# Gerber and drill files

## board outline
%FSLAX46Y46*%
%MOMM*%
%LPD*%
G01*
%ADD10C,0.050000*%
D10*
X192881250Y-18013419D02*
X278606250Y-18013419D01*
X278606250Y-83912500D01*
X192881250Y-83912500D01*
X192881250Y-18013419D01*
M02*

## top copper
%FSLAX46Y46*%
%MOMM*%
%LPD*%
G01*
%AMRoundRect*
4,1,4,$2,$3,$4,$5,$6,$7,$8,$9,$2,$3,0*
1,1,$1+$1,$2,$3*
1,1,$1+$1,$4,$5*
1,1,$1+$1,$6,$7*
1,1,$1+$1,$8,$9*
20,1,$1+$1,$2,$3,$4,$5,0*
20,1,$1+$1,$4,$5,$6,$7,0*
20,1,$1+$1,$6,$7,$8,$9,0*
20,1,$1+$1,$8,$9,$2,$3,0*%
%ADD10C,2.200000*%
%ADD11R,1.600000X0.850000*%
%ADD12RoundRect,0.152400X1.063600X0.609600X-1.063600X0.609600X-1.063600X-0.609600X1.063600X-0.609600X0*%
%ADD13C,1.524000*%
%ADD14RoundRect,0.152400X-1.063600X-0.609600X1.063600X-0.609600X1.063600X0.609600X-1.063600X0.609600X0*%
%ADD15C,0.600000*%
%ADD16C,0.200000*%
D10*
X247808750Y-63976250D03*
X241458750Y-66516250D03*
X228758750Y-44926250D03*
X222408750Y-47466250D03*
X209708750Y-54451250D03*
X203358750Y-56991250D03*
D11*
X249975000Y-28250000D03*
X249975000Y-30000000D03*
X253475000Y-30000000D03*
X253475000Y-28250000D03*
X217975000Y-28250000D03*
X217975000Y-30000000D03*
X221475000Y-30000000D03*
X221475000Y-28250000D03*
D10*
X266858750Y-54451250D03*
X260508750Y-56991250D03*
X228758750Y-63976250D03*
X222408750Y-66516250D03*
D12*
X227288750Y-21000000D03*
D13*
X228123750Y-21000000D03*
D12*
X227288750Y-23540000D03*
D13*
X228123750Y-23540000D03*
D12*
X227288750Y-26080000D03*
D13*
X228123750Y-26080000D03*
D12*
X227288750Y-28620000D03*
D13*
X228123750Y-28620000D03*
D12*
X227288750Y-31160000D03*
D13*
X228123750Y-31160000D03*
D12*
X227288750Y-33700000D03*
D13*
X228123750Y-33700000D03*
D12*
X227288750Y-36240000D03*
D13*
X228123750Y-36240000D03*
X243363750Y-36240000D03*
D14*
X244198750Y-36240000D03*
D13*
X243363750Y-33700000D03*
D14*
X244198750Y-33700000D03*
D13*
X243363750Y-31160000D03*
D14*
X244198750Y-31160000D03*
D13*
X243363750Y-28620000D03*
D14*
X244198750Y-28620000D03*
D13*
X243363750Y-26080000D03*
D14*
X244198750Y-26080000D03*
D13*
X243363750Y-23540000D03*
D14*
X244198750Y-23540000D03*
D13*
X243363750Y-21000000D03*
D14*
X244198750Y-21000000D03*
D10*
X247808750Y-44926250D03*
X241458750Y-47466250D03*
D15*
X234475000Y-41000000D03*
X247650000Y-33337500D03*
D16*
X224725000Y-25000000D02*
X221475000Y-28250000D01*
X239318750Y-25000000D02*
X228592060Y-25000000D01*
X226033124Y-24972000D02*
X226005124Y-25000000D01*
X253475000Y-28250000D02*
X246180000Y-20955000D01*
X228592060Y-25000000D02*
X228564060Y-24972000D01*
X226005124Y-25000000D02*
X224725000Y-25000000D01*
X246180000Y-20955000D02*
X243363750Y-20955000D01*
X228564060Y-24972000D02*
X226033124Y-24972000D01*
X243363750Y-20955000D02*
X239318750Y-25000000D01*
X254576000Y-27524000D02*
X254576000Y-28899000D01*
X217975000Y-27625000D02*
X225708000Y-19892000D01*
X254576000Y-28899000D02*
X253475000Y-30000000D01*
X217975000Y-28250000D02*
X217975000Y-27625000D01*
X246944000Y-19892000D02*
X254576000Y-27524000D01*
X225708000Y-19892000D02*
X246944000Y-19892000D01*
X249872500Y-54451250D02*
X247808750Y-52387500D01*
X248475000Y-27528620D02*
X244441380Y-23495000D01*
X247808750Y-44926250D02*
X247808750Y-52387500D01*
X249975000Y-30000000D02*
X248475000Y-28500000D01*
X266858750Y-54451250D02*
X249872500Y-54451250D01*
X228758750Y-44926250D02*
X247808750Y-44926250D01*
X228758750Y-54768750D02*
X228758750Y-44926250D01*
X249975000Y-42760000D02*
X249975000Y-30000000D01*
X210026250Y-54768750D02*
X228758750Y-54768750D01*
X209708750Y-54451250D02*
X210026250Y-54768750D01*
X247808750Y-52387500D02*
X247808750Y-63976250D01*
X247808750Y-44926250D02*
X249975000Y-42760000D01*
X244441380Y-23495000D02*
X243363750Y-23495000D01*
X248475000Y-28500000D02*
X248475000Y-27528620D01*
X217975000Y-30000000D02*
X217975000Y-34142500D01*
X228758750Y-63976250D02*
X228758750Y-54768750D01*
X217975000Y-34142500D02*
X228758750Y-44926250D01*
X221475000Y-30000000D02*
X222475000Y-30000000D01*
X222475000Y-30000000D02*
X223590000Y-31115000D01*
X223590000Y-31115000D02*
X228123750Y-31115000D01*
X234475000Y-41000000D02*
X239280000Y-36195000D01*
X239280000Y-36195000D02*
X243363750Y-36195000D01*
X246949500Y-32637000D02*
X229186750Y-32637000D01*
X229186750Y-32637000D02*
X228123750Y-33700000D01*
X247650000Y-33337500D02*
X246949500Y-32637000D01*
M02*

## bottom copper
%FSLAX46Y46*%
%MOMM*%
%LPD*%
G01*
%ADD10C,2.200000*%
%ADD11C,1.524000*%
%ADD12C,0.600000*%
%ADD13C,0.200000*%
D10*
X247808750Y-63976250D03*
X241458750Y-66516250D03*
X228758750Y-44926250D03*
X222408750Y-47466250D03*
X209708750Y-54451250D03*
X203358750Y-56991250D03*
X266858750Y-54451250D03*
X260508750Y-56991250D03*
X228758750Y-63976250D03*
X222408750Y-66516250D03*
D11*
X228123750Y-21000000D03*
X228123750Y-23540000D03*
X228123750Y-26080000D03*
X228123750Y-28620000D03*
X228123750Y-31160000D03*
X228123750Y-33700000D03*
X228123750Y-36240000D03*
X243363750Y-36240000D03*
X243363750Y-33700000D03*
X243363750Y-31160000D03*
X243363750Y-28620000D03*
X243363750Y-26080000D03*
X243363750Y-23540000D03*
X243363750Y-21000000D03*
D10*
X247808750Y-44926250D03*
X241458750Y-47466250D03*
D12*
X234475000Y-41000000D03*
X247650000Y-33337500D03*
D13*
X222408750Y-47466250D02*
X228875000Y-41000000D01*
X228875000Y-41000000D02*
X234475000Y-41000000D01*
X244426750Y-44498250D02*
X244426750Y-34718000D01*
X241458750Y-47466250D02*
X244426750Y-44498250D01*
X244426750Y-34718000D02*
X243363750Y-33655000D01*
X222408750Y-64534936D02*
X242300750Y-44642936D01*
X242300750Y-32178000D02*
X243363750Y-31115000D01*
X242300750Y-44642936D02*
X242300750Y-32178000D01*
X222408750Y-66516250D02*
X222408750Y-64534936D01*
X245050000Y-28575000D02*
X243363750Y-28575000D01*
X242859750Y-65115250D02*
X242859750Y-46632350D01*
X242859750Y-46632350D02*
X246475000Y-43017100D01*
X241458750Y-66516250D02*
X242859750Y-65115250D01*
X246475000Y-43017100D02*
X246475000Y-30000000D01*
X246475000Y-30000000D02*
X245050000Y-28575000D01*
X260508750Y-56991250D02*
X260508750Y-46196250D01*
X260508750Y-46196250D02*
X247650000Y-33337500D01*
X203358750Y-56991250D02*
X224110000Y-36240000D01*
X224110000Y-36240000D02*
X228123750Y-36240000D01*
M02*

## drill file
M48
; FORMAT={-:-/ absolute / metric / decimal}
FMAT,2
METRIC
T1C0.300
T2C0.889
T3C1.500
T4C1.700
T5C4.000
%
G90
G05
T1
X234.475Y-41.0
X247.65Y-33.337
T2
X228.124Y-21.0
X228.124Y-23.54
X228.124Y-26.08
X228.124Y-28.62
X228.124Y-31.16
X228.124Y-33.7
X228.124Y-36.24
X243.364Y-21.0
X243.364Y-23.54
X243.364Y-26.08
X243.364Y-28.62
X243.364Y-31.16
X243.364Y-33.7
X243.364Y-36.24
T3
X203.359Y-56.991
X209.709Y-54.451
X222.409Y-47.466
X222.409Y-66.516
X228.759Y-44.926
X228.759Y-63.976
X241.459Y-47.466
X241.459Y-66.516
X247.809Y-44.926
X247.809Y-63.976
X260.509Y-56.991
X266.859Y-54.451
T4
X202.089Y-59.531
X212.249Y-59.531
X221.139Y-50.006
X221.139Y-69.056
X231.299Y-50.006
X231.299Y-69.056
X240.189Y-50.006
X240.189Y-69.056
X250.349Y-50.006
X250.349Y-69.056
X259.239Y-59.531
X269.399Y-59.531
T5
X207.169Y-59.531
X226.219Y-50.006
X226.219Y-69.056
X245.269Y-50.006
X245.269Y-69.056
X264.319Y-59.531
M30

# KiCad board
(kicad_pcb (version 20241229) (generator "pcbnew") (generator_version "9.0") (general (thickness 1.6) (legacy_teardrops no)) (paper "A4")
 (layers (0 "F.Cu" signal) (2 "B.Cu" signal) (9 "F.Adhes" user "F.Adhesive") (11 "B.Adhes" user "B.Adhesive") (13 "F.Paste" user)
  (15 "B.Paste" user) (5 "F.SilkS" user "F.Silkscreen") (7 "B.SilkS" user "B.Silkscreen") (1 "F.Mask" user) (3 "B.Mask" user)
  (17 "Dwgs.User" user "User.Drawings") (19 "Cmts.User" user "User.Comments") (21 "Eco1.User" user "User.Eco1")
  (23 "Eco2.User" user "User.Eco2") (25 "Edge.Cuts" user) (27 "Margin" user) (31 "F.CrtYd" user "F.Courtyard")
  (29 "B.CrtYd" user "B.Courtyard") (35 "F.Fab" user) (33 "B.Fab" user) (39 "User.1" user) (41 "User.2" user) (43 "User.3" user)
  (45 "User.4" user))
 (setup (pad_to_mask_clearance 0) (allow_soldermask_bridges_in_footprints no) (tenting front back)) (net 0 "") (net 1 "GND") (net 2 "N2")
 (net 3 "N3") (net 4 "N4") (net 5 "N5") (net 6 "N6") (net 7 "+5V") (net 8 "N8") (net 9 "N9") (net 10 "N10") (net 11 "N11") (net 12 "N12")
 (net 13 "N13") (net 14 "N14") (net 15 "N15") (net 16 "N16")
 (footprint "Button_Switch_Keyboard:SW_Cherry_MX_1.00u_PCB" (layer "F.Cu") (at 247.80875 63.97625)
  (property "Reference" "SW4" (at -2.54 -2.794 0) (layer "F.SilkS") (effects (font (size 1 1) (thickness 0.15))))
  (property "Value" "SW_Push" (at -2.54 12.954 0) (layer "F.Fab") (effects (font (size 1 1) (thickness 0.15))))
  (pad "" np_thru_hole circle (at -7.62 5.08) (size 1.7 1.7) (drill 1.7) (layers "*.Cu" "*.Mask"))
  (pad "" np_thru_hole circle (at -2.54 5.08) (size 4 4) (drill 4) (layers "*.Cu" "*.Mask"))
  (pad "" np_thru_hole circle (at 2.54 5.08) (size 1.7 1.7) (drill 1.7) (layers "*.Cu" "*.Mask"))
  (pad "1" thru_hole circle (at 0 0) (size 2.2 2.2) (drill 1.5) (layers "*.Cu" "*.Mask") (remove_unused_layers no) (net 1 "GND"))
  (pad "2" thru_hole circle (at -6.35 2.54) (size 2.2 2.2) (drill 1.5) (layers "*.Cu" "*.Mask") (remove_unused_layers no) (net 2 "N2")))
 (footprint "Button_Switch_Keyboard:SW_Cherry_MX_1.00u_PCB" (layer "F.Cu") (at 228.75875 44.92625)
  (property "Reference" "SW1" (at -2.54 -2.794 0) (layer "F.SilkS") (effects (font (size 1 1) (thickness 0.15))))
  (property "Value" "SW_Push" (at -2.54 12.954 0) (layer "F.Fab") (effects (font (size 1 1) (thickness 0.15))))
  (pad "" np_thru_hole circle (at -7.62 5.08) (size 1.7 1.7) (drill 1.7) (layers "*.Cu" "*.Mask"))
  (pad "" np_thru_hole circle (at -2.54 5.08) (size 4 4) (drill 4) (layers "*.Cu" "*.Mask"))
  (pad "" np_thru_hole circle (at 2.54 5.08) (size 1.7 1.7) (drill 1.7) (layers "*.Cu" "*.Mask"))
  (pad "1" thru_hole circle (at 0 0) (size 2.2 2.2) (drill 1.5) (layers "*.Cu" "*.Mask") (remove_unused_layers no) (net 1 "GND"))
  (pad "2" thru_hole circle (at -6.35 2.54) (size 2.2 2.2) (drill 1.5) (layers "*.Cu" "*.Mask") (remove_unused_layers no) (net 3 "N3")))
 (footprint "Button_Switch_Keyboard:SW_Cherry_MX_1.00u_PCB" (layer "F.Cu") (at 209.70875 54.45125)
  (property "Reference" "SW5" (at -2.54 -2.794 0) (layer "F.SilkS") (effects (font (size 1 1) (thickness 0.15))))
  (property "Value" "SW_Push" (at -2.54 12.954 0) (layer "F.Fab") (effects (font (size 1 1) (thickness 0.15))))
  (pad "" np_thru_hole circle (at -7.62 5.08) (size 1.7 1.7) (drill 1.7) (layers "*.Cu" "*.Mask"))
  (pad "" np_thru_hole circle (at -2.54 5.08) (size 4 4) (drill 4) (layers "*.Cu" "*.Mask"))
  (pad "" np_thru_hole circle (at 2.54 5.08) (size 1.7 1.7) (drill 1.7) (layers "*.Cu" "*.Mask"))
  (pad "1" thru_hole circle (at 0 0) (size 2.2 2.2) (drill 1.5) (layers "*.Cu" "*.Mask") (remove_unused_layers no) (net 1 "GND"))
  (pad "2" thru_hole circle (at -6.35 2.54) (size 2.2 2.2) (drill 1.5) (layers "*.Cu" "*.Mask") (remove_unused_layers no) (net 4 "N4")))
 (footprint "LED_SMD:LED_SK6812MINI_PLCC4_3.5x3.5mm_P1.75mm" (layer "F.Cu") (at 251.725 29.125)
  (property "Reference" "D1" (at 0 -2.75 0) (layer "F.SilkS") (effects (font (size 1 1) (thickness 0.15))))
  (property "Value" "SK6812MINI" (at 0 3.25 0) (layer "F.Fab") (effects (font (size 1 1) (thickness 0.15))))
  (pad "1" smd rect (at -1.75 -0.875) (size 1.6 0.85) (layers "F.Cu" "F.Mask" "F.Paste") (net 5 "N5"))
  (pad "2" smd rect (at -1.75 0.875) (size 1.6 0.85) (layers "F.Cu" "F.Mask" "F.Paste") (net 1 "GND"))
  (pad "3" smd rect (at 1.75 0.875) (size 1.6 0.85) (layers "F.Cu" "F.Mask" "F.Paste") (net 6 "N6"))
  (pad "4" smd rect (at 1.75 -0.875) (size 1.6 0.85) (layers "F.Cu" "F.Mask" "F.Paste") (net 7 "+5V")))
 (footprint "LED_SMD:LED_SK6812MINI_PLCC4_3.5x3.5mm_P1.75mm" (layer "F.Cu") (at 219.725 29.125)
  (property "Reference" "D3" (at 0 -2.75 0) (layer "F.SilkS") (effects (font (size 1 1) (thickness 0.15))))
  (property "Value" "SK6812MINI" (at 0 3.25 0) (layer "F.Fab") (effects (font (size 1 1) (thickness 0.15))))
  (pad "1" smd rect (at -1.75 -0.875) (size 1.6 0.85) (layers "F.Cu" "F.Mask" "F.Paste") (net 6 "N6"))
  (pad "2" smd rect (at -1.75 0.875) (size 1.6 0.85) (layers "F.Cu" "F.Mask" "F.Paste") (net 1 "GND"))
  (pad "3" smd rect (at 1.75 0.875) (size 1.6 0.85) (layers "F.Cu" "F.Mask" "F.Paste") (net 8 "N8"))
  (pad "4" smd rect (at 1.75 -0.875) (size 1.6 0.85) (layers "F.Cu" "F.Mask" "F.Paste") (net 7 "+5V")))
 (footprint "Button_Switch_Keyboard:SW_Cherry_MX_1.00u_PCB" (layer "F.Cu") (at 266.85875 54.45125)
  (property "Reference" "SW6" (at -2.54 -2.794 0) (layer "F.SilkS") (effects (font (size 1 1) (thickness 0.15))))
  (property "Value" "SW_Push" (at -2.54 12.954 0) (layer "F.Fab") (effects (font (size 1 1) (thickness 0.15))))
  (pad "" np_thru_hole circle (at -7.62 5.08) (size 1.7 1.7) (drill 1.7) (layers "*.Cu" "*.Mask"))
  (pad "" np_thru_hole circle (at -2.54 5.08) (size 4 4) (drill 4) (layers "*.Cu" "*.Mask"))
  (pad "" np_thru_hole circle (at 2.54 5.08) (size 1.7 1.7) (drill 1.7) (layers "*.Cu" "*.Mask"))
  (pad "1" thru_hole circle (at 0 0) (size 2.2 2.2) (drill 1.5) (layers "*.Cu" "*.Mask") (remove_unused_layers no) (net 1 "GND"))
  (pad "2" thru_hole circle (at -6.35 2.54) (size 2.2 2.2) (drill 1.5) (layers "*.Cu" "*.Mask") (remove_unused_layers no) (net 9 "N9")))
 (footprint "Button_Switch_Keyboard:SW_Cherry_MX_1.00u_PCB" (layer "F.Cu") (at 228.75875 63.97625)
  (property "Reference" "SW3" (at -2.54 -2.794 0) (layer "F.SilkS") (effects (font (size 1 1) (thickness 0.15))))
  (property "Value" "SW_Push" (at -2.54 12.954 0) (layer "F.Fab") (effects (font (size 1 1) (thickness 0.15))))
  (pad "" np_thru_hole circle (at -7.62 5.08) (size 1.7 1.7) (drill 1.7) (layers "*.Cu" "*.Mask"))
  (pad "" np_thru_hole circle (at -2.54 5.08) (size 4 4) (drill 4) (layers "*.Cu" "*.Mask"))
  (pad "" np_thru_hole circle (at 2.54 5.08) (size 1.7 1.7) (drill 1.7) (layers "*.Cu" "*.Mask"))
  (pad "1" thru_hole circle (at 0 0) (size 2.2 2.2) (drill 1.5) (layers "*.Cu" "*.Mask") (remove_unused_layers no) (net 1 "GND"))
  (pad "2" thru_hole circle (at -6.35 2.54) (size 2.2 2.2) (drill 1.5) (layers "*.Cu" "*.Mask") (remove_unused_layers no) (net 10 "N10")))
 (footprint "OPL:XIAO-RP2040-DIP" (layer "F.Cu") (at 235.74375 28.62)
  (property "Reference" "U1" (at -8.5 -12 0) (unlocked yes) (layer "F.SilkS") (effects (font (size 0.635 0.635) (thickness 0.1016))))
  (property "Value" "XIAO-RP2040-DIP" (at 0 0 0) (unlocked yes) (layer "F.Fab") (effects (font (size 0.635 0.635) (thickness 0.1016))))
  (pad "1" smd roundrect (at -8.455 -7.62 180) (size 2.432 1.524) (layers "F.Cu" "F.Mask") (roundrect_rratio 0.1) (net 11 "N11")
   (thermal_bridge_angle 45))
  (pad "1" thru_hole circle (at -7.62 -7.62 180) (size 1.524 1.524) (drill 0.889) (layers "*.Cu" "*.Mask") (remove_unused_layers no)
   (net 11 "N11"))
  (pad "2" smd roundrect (at -8.455 -5.08 180) (size 2.432 1.524) (layers "F.Cu" "F.Mask") (roundrect_rratio 0.1) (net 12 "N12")
   (thermal_bridge_angle 45))
  (pad "2" thru_hole circle (at -7.62 -5.08 180) (size 1.524 1.524) (drill 0.889) (layers "*.Cu" "*.Mask") (remove_unused_layers no)
   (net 12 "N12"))
  (pad "3" smd roundrect (at -8.455 -2.54 180) (size 2.432 1.524) (layers "F.Cu" "F.Mask") (roundrect_rratio 0.1) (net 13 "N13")
   (thermal_bridge_angle 45))
  (pad "3" thru_hole circle (at -7.62 -2.54 180) (size 1.524 1.524) (drill 0.889) (layers "*.Cu" "*.Mask") (remove_unused_layers no)
   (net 13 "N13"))
  (pad "4" smd roundrect (at -8.455 0 180) (size 2.432 1.524) (layers "F.Cu" "F.Mask") (roundrect_rratio 0.1) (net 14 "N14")
   (thermal_bridge_angle 45))
  (pad "4" thru_hole circle (at -7.62 0 180) (size 1.524 1.524) (drill 0.889) (layers "*.Cu" "*.Mask") (remove_unused_layers no)
   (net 14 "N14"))
  (pad "5" smd roundrect (at -8.455 2.54 180) (size 2.432 1.524) (layers "F.Cu" "F.Mask") (roundrect_rratio 0.1) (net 8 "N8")
   (thermal_bridge_angle 45))
  (pad "5" thru_hole circle (at -7.62 2.54 180) (size 1.524 1.524) (drill 0.889) (layers "*.Cu" "*.Mask") (remove_unused_layers no)
   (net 8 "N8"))
  (pad "6" smd roundrect (at -8.455 5.08 180) (size 2.432 1.524) (layers "F.Cu" "F.Mask") (roundrect_rratio 0.1) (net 9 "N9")
   (thermal_bridge_angle 45))
  (pad "6" thru_hole circle (at -7.62 5.08 180) (size 1.524 1.524) (drill 0.889) (layers "*.Cu" "*.Mask") (remove_unused_layers no)
   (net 9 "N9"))
  (pad "7" smd roundrect (at -8.455 7.62 180) (size 2.432 1.524) (layers "F.Cu" "F.Mask") (roundrect_rratio 0.1) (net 4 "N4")
   (thermal_bridge_angle 45))
  (pad "7" thru_hole circle (at -7.62 7.62 180) (size 1.524 1.524) (drill 0.889) (layers "*.Cu" "*.Mask") (remove_unused_layers no)
   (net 4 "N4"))
  (pad "8" thru_hole circle (at 7.62 7.62) (size 1.524 1.524) (drill 0.889) (layers "*.Cu" "*.Mask") (remove_unused_layers no) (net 3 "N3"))
  (pad "8" smd roundrect (at 8.455 7.62) (size 2.432 1.524) (layers "F.Cu" "F.Mask") (roundrect_rratio 0.1) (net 3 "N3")
   (thermal_bridge_angle 45))
  (pad "9" thru_hole circle (at 7.62 5.08) (size 1.524 1.524) (drill 0.889) (layers "*.Cu" "*.Mask") (remove_unused_layers no)
   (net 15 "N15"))
  (pad "9" smd roundrect (at 8.455 5.08) (size 2.432 1.524) (layers "F.Cu" "F.Mask") (roundrect_rratio 0.1) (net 15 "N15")
   (thermal_bridge_angle 45))
  (pad "10" thru_hole circle (at 7.62 2.54) (size 1.524 1.524) (drill 0.889) (layers "*.Cu" "*.Mask") (remove_unused_layers no)
   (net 10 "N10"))
  (pad "10" smd roundrect (at 8.455 2.54) (size 2.432 1.524) (layers "F.Cu" "F.Mask") (roundrect_rratio 0.1) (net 10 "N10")
   (thermal_bridge_angle 45))
  (pad "11" thru_hole circle (at 7.62 0) (size 1.524 1.524) (drill 0.889) (layers "*.Cu" "*.Mask") (remove_unused_layers no) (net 2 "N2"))
  (pad "11" smd roundrect (at 8.455 0) (size 2.432 1.524) (layers "F.Cu" "F.Mask") (roundrect_rratio 0.1) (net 2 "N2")
   (thermal_bridge_angle 45))
  (pad "12" thru_hole circle (at 7.62 -2.54) (size 1.524 1.524) (drill 0.889) (layers "*.Cu" "*.Mask") (remove_unused_layers no)
   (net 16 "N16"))
  (pad "12" smd roundrect (at 8.455 -2.54) (size 2.432 1.524) (layers "F.Cu" "F.Mask") (roundrect_rratio 0.1) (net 16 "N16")
   (thermal_bridge_angle 45))
  (pad "13" thru_hole circle (at 7.62 -5.08) (size 1.524 1.524) (drill 0.889) (layers "*.Cu" "*.Mask") (remove_unused_layers no)
   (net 1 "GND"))
  (pad "13" smd roundrect (at 8.455 -5.08) (size 2.432 1.524) (layers "F.Cu" "F.Mask") (roundrect_rratio 0.1) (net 1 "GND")
   (thermal_bridge_angle 45))
  (pad "14" thru_hole circle (at 7.62 -7.62) (size 1.524 1.524) (drill 0.889) (layers "*.Cu" "*.Mask") (remove_unused_layers no)
   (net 7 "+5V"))
  (pad "14" smd roundrect (at 8.455 -7.62) (size 2.432 1.524) (layers "F.Cu" "F.Mask") (roundrect_rratio 0.1) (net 7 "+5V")
   (thermal_bridge_angle 45)))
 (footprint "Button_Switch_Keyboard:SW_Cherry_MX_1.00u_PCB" (layer "F.Cu") (at 247.80875 44.92625)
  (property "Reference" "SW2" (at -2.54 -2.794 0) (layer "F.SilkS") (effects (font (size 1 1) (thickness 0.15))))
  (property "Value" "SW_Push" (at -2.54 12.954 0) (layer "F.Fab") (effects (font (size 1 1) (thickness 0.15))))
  (pad "" np_thru_hole circle (at -7.62 5.08) (size 1.7 1.7) (drill 1.7) (layers "*.Cu" "*.Mask"))
  (pad "" np_thru_hole circle (at -2.54 5.08) (size 4 4) (drill 4) (layers "*.Cu" "*.Mask"))
  (pad "" np_thru_hole circle (at 2.54 5.08) (size 1.7 1.7) (drill 1.7) (layers "*.Cu" "*.Mask"))
  (pad "1" thru_hole circle (at 0 0) (size 2.2 2.2) (drill 1.5) (layers "*.Cu" "*.Mask") (remove_unused_layers no) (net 1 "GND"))
  (pad "2" thru_hole circle (at -6.35 2.54) (size 2.2 2.2) (drill 1.5) (layers "*.Cu" "*.Mask") (remove_unused_layers no) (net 15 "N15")))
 (gr_rect (start 192.88125 18.013419) (end 278.60625 83.9125) (stroke (width 0.05) (type default)) (fill no) (layer "Edge.Cuts"))
 (segment (start 224.725 25) (end 221.475 28.25) (width 0.2) (layer "F.Cu") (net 7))
 (segment (start 239.31875 25) (end 228.59206 25) (width 0.2) (layer "F.Cu") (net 7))
 (segment (start 226.033124 24.972) (end 226.005124 25) (width 0.2) (layer "F.Cu") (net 7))
 (segment (start 253.475 28.25) (end 246.18 20.955) (width 0.2) (layer "F.Cu") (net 7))
 (segment (start 228.59206 25) (end 228.56406 24.972) (width 0.2) (layer "F.Cu") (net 7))
 (segment (start 226.005124 25) (end 224.725 25) (width 0.2) (layer "F.Cu") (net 7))
 (segment (start 246.18 20.955) (end 243.36375 20.955) (width 0.2) (layer "F.Cu") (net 7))
 (segment (start 228.56406 24.972) (end 226.033124 24.972) (width 0.2) (layer "F.Cu") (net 7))
 (segment (start 243.36375 20.955) (end 239.31875 25) (width 0.2) (layer "F.Cu") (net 7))
 (segment (start 254.576 27.524) (end 254.576 28.899) (width 0.2) (layer "F.Cu") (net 6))
 (segment (start 217.975 27.625) (end 225.708 19.892) (width 0.2) (layer "F.Cu") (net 6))
 (segment (start 254.576 28.899) (end 253.475 30) (width 0.2) (layer "F.Cu") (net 6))
 (segment (start 217.975 28.25) (end 217.975 27.625) (width 0.2) (layer "F.Cu") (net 6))
 (segment (start 246.944 19.892) (end 254.576 27.524) (width 0.2) (layer "F.Cu") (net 6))
 (segment (start 225.708 19.892) (end 246.944 19.892) (width 0.2) (layer "F.Cu") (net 6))
 (segment (start 249.8725 54.45125) (end 247.80875 52.3875) (width 0.2) (layer "F.Cu") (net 1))
 (segment (start 248.475 27.52862) (end 244.44138 23.495) (width 0.2) (layer "F.Cu") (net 1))
 (segment (start 247.80875 44.92625) (end 247.80875 52.3875) (width 0.2) (layer "F.Cu") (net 1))
 (segment (start 249.975 30) (end 248.475 28.5) (width 0.2) (layer "F.Cu") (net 1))
 (segment (start 266.85875 54.45125) (end 249.8725 54.45125) (width 0.2) (layer "F.Cu") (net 1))
 (segment (start 228.75875 44.92625) (end 247.80875 44.92625) (width 0.2) (layer "F.Cu") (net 1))
 (segment (start 228.75875 54.76875) (end 228.75875 44.92625) (width 0.2) (layer "F.Cu") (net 1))
 (segment (start 249.975 42.76) (end 249.975 30) (width 0.2) (layer "F.Cu") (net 1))
 (segment (start 210.02625 54.76875) (end 228.75875 54.76875) (width 0.2) (layer "F.Cu") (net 1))
 (segment (start 209.70875 54.45125) (end 210.02625 54.76875) (width 0.2) (layer "F.Cu") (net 1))
 (segment (start 247.80875 52.3875) (end 247.80875 63.97625) (width 0.2) (layer "F.Cu") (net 1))
 (segment (start 247.80875 44.92625) (end 249.975 42.76) (width 0.2) (layer "F.Cu") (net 1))
 (segment (start 244.44138 23.495) (end 243.36375 23.495) (width 0.2) (layer "F.Cu") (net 1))
 (segment (start 248.475 28.5) (end 248.475 27.52862) (width 0.2) (layer "F.Cu") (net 1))
 (segment (start 217.975 30) (end 217.975 34.1425) (width 0.2) (layer "F.Cu") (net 1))
 (segment (start 228.75875 63.97625) (end 228.75875 54.76875) (width 0.2) (layer "F.Cu") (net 1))
 (segment (start 217.975 34.1425) (end 228.75875 44.92625) (width 0.2) (layer "F.Cu") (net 1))
 (segment (start 221.475 30) (end 222.475 30) (width 0.2) (layer "F.Cu") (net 8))
 (segment (start 222.475 30) (end 223.59 31.115) (width 0.2) (layer "F.Cu") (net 8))
 (segment (start 223.59 31.115) (end 228.12375 31.115) (width 0.2) (layer "F.Cu") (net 8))
 (segment (start 234.475 41) (end 239.28 36.195) (width 0.2) (layer "F.Cu") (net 3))
 (segment (start 239.28 36.195) (end 243.36375 36.195) (width 0.2) (layer "F.Cu") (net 3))
 (via (at 234.475 41) (size 0.6) (drill 0.3) (layers "F.Cu" "B.Cu") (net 3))
 (segment (start 222.40875 47.46625) (end 228.875 41) (width 0.2) (layer "B.Cu") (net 3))
 (segment (start 228.875 41) (end 234.475 41) (width 0.2) (layer "B.Cu") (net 3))
 (segment (start 244.42675 44.49825) (end 244.42675 34.718) (width 0.2) (layer "B.Cu") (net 15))
 (segment (start 241.45875 47.46625) (end 244.42675 44.49825) (width 0.2) (layer "B.Cu") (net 15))
 (segment (start 244.42675 34.718) (end 243.36375 33.655) (width 0.2) (layer "B.Cu") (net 15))
 (segment (start 222.40875 64.534936) (end 242.30075 44.642936) (width 0.2) (layer "B.Cu") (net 10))
 (segment (start 242.30075 32.178) (end 243.36375 31.115) (width 0.2) (layer "B.Cu") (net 10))
 (segment (start 242.30075 44.642936) (end 242.30075 32.178) (width 0.2) (layer "B.Cu") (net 10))
 (segment (start 222.40875 66.51625) (end 222.40875 64.534936) (width 0.2) (layer "B.Cu") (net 10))
 (segment (start 245.05 28.575) (end 243.36375 28.575) (width 0.2) (layer "B.Cu") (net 2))
 (segment (start 242.85975 65.11525) (end 242.85975 46.63235) (width 0.2) (layer "B.Cu") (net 2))
 (segment (start 242.85975 46.63235) (end 246.475 43.0171) (width 0.2) (layer "B.Cu") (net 2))
 (segment (start 241.45875 66.51625) (end 242.85975 65.11525) (width 0.2) (layer "B.Cu") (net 2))
 (segment (start 246.475 43.0171) (end 246.475 30) (width 0.2) (layer "B.Cu") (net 2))
 (segment (start 246.475 30) (end 245.05 28.575) (width 0.2) (layer "B.Cu") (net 2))
 (segment (start 246.9495 32.637) (end 229.18675 32.637) (width 0.2) (layer "F.Cu") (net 9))
 (segment (start 229.18675 32.637) (end 228.12375 33.7) (width 0.2) (layer "F.Cu") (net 9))
 (segment (start 247.65 33.3375) (end 246.9495 32.637) (width 0.2) (layer "F.Cu") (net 9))
 (via (at 247.65 33.3375) (size 0.6) (drill 0.3) (layers "F.Cu" "B.Cu") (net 9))
 (segment (start 260.50875 56.99125) (end 260.50875 46.19625) (width 0.2) (layer "B.Cu") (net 9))
 (segment (start 260.50875 46.19625) (end 247.65 33.3375) (width 0.2) (layer "B.Cu") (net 9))
 (segment (start 203.35875 56.99125) (end 224.11 36.24) (width 0.2) (layer "B.Cu") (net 4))
 (segment (start 224.11 36.24) (end 228.12375 36.24) (width 0.2) (layer "B.Cu") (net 4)))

